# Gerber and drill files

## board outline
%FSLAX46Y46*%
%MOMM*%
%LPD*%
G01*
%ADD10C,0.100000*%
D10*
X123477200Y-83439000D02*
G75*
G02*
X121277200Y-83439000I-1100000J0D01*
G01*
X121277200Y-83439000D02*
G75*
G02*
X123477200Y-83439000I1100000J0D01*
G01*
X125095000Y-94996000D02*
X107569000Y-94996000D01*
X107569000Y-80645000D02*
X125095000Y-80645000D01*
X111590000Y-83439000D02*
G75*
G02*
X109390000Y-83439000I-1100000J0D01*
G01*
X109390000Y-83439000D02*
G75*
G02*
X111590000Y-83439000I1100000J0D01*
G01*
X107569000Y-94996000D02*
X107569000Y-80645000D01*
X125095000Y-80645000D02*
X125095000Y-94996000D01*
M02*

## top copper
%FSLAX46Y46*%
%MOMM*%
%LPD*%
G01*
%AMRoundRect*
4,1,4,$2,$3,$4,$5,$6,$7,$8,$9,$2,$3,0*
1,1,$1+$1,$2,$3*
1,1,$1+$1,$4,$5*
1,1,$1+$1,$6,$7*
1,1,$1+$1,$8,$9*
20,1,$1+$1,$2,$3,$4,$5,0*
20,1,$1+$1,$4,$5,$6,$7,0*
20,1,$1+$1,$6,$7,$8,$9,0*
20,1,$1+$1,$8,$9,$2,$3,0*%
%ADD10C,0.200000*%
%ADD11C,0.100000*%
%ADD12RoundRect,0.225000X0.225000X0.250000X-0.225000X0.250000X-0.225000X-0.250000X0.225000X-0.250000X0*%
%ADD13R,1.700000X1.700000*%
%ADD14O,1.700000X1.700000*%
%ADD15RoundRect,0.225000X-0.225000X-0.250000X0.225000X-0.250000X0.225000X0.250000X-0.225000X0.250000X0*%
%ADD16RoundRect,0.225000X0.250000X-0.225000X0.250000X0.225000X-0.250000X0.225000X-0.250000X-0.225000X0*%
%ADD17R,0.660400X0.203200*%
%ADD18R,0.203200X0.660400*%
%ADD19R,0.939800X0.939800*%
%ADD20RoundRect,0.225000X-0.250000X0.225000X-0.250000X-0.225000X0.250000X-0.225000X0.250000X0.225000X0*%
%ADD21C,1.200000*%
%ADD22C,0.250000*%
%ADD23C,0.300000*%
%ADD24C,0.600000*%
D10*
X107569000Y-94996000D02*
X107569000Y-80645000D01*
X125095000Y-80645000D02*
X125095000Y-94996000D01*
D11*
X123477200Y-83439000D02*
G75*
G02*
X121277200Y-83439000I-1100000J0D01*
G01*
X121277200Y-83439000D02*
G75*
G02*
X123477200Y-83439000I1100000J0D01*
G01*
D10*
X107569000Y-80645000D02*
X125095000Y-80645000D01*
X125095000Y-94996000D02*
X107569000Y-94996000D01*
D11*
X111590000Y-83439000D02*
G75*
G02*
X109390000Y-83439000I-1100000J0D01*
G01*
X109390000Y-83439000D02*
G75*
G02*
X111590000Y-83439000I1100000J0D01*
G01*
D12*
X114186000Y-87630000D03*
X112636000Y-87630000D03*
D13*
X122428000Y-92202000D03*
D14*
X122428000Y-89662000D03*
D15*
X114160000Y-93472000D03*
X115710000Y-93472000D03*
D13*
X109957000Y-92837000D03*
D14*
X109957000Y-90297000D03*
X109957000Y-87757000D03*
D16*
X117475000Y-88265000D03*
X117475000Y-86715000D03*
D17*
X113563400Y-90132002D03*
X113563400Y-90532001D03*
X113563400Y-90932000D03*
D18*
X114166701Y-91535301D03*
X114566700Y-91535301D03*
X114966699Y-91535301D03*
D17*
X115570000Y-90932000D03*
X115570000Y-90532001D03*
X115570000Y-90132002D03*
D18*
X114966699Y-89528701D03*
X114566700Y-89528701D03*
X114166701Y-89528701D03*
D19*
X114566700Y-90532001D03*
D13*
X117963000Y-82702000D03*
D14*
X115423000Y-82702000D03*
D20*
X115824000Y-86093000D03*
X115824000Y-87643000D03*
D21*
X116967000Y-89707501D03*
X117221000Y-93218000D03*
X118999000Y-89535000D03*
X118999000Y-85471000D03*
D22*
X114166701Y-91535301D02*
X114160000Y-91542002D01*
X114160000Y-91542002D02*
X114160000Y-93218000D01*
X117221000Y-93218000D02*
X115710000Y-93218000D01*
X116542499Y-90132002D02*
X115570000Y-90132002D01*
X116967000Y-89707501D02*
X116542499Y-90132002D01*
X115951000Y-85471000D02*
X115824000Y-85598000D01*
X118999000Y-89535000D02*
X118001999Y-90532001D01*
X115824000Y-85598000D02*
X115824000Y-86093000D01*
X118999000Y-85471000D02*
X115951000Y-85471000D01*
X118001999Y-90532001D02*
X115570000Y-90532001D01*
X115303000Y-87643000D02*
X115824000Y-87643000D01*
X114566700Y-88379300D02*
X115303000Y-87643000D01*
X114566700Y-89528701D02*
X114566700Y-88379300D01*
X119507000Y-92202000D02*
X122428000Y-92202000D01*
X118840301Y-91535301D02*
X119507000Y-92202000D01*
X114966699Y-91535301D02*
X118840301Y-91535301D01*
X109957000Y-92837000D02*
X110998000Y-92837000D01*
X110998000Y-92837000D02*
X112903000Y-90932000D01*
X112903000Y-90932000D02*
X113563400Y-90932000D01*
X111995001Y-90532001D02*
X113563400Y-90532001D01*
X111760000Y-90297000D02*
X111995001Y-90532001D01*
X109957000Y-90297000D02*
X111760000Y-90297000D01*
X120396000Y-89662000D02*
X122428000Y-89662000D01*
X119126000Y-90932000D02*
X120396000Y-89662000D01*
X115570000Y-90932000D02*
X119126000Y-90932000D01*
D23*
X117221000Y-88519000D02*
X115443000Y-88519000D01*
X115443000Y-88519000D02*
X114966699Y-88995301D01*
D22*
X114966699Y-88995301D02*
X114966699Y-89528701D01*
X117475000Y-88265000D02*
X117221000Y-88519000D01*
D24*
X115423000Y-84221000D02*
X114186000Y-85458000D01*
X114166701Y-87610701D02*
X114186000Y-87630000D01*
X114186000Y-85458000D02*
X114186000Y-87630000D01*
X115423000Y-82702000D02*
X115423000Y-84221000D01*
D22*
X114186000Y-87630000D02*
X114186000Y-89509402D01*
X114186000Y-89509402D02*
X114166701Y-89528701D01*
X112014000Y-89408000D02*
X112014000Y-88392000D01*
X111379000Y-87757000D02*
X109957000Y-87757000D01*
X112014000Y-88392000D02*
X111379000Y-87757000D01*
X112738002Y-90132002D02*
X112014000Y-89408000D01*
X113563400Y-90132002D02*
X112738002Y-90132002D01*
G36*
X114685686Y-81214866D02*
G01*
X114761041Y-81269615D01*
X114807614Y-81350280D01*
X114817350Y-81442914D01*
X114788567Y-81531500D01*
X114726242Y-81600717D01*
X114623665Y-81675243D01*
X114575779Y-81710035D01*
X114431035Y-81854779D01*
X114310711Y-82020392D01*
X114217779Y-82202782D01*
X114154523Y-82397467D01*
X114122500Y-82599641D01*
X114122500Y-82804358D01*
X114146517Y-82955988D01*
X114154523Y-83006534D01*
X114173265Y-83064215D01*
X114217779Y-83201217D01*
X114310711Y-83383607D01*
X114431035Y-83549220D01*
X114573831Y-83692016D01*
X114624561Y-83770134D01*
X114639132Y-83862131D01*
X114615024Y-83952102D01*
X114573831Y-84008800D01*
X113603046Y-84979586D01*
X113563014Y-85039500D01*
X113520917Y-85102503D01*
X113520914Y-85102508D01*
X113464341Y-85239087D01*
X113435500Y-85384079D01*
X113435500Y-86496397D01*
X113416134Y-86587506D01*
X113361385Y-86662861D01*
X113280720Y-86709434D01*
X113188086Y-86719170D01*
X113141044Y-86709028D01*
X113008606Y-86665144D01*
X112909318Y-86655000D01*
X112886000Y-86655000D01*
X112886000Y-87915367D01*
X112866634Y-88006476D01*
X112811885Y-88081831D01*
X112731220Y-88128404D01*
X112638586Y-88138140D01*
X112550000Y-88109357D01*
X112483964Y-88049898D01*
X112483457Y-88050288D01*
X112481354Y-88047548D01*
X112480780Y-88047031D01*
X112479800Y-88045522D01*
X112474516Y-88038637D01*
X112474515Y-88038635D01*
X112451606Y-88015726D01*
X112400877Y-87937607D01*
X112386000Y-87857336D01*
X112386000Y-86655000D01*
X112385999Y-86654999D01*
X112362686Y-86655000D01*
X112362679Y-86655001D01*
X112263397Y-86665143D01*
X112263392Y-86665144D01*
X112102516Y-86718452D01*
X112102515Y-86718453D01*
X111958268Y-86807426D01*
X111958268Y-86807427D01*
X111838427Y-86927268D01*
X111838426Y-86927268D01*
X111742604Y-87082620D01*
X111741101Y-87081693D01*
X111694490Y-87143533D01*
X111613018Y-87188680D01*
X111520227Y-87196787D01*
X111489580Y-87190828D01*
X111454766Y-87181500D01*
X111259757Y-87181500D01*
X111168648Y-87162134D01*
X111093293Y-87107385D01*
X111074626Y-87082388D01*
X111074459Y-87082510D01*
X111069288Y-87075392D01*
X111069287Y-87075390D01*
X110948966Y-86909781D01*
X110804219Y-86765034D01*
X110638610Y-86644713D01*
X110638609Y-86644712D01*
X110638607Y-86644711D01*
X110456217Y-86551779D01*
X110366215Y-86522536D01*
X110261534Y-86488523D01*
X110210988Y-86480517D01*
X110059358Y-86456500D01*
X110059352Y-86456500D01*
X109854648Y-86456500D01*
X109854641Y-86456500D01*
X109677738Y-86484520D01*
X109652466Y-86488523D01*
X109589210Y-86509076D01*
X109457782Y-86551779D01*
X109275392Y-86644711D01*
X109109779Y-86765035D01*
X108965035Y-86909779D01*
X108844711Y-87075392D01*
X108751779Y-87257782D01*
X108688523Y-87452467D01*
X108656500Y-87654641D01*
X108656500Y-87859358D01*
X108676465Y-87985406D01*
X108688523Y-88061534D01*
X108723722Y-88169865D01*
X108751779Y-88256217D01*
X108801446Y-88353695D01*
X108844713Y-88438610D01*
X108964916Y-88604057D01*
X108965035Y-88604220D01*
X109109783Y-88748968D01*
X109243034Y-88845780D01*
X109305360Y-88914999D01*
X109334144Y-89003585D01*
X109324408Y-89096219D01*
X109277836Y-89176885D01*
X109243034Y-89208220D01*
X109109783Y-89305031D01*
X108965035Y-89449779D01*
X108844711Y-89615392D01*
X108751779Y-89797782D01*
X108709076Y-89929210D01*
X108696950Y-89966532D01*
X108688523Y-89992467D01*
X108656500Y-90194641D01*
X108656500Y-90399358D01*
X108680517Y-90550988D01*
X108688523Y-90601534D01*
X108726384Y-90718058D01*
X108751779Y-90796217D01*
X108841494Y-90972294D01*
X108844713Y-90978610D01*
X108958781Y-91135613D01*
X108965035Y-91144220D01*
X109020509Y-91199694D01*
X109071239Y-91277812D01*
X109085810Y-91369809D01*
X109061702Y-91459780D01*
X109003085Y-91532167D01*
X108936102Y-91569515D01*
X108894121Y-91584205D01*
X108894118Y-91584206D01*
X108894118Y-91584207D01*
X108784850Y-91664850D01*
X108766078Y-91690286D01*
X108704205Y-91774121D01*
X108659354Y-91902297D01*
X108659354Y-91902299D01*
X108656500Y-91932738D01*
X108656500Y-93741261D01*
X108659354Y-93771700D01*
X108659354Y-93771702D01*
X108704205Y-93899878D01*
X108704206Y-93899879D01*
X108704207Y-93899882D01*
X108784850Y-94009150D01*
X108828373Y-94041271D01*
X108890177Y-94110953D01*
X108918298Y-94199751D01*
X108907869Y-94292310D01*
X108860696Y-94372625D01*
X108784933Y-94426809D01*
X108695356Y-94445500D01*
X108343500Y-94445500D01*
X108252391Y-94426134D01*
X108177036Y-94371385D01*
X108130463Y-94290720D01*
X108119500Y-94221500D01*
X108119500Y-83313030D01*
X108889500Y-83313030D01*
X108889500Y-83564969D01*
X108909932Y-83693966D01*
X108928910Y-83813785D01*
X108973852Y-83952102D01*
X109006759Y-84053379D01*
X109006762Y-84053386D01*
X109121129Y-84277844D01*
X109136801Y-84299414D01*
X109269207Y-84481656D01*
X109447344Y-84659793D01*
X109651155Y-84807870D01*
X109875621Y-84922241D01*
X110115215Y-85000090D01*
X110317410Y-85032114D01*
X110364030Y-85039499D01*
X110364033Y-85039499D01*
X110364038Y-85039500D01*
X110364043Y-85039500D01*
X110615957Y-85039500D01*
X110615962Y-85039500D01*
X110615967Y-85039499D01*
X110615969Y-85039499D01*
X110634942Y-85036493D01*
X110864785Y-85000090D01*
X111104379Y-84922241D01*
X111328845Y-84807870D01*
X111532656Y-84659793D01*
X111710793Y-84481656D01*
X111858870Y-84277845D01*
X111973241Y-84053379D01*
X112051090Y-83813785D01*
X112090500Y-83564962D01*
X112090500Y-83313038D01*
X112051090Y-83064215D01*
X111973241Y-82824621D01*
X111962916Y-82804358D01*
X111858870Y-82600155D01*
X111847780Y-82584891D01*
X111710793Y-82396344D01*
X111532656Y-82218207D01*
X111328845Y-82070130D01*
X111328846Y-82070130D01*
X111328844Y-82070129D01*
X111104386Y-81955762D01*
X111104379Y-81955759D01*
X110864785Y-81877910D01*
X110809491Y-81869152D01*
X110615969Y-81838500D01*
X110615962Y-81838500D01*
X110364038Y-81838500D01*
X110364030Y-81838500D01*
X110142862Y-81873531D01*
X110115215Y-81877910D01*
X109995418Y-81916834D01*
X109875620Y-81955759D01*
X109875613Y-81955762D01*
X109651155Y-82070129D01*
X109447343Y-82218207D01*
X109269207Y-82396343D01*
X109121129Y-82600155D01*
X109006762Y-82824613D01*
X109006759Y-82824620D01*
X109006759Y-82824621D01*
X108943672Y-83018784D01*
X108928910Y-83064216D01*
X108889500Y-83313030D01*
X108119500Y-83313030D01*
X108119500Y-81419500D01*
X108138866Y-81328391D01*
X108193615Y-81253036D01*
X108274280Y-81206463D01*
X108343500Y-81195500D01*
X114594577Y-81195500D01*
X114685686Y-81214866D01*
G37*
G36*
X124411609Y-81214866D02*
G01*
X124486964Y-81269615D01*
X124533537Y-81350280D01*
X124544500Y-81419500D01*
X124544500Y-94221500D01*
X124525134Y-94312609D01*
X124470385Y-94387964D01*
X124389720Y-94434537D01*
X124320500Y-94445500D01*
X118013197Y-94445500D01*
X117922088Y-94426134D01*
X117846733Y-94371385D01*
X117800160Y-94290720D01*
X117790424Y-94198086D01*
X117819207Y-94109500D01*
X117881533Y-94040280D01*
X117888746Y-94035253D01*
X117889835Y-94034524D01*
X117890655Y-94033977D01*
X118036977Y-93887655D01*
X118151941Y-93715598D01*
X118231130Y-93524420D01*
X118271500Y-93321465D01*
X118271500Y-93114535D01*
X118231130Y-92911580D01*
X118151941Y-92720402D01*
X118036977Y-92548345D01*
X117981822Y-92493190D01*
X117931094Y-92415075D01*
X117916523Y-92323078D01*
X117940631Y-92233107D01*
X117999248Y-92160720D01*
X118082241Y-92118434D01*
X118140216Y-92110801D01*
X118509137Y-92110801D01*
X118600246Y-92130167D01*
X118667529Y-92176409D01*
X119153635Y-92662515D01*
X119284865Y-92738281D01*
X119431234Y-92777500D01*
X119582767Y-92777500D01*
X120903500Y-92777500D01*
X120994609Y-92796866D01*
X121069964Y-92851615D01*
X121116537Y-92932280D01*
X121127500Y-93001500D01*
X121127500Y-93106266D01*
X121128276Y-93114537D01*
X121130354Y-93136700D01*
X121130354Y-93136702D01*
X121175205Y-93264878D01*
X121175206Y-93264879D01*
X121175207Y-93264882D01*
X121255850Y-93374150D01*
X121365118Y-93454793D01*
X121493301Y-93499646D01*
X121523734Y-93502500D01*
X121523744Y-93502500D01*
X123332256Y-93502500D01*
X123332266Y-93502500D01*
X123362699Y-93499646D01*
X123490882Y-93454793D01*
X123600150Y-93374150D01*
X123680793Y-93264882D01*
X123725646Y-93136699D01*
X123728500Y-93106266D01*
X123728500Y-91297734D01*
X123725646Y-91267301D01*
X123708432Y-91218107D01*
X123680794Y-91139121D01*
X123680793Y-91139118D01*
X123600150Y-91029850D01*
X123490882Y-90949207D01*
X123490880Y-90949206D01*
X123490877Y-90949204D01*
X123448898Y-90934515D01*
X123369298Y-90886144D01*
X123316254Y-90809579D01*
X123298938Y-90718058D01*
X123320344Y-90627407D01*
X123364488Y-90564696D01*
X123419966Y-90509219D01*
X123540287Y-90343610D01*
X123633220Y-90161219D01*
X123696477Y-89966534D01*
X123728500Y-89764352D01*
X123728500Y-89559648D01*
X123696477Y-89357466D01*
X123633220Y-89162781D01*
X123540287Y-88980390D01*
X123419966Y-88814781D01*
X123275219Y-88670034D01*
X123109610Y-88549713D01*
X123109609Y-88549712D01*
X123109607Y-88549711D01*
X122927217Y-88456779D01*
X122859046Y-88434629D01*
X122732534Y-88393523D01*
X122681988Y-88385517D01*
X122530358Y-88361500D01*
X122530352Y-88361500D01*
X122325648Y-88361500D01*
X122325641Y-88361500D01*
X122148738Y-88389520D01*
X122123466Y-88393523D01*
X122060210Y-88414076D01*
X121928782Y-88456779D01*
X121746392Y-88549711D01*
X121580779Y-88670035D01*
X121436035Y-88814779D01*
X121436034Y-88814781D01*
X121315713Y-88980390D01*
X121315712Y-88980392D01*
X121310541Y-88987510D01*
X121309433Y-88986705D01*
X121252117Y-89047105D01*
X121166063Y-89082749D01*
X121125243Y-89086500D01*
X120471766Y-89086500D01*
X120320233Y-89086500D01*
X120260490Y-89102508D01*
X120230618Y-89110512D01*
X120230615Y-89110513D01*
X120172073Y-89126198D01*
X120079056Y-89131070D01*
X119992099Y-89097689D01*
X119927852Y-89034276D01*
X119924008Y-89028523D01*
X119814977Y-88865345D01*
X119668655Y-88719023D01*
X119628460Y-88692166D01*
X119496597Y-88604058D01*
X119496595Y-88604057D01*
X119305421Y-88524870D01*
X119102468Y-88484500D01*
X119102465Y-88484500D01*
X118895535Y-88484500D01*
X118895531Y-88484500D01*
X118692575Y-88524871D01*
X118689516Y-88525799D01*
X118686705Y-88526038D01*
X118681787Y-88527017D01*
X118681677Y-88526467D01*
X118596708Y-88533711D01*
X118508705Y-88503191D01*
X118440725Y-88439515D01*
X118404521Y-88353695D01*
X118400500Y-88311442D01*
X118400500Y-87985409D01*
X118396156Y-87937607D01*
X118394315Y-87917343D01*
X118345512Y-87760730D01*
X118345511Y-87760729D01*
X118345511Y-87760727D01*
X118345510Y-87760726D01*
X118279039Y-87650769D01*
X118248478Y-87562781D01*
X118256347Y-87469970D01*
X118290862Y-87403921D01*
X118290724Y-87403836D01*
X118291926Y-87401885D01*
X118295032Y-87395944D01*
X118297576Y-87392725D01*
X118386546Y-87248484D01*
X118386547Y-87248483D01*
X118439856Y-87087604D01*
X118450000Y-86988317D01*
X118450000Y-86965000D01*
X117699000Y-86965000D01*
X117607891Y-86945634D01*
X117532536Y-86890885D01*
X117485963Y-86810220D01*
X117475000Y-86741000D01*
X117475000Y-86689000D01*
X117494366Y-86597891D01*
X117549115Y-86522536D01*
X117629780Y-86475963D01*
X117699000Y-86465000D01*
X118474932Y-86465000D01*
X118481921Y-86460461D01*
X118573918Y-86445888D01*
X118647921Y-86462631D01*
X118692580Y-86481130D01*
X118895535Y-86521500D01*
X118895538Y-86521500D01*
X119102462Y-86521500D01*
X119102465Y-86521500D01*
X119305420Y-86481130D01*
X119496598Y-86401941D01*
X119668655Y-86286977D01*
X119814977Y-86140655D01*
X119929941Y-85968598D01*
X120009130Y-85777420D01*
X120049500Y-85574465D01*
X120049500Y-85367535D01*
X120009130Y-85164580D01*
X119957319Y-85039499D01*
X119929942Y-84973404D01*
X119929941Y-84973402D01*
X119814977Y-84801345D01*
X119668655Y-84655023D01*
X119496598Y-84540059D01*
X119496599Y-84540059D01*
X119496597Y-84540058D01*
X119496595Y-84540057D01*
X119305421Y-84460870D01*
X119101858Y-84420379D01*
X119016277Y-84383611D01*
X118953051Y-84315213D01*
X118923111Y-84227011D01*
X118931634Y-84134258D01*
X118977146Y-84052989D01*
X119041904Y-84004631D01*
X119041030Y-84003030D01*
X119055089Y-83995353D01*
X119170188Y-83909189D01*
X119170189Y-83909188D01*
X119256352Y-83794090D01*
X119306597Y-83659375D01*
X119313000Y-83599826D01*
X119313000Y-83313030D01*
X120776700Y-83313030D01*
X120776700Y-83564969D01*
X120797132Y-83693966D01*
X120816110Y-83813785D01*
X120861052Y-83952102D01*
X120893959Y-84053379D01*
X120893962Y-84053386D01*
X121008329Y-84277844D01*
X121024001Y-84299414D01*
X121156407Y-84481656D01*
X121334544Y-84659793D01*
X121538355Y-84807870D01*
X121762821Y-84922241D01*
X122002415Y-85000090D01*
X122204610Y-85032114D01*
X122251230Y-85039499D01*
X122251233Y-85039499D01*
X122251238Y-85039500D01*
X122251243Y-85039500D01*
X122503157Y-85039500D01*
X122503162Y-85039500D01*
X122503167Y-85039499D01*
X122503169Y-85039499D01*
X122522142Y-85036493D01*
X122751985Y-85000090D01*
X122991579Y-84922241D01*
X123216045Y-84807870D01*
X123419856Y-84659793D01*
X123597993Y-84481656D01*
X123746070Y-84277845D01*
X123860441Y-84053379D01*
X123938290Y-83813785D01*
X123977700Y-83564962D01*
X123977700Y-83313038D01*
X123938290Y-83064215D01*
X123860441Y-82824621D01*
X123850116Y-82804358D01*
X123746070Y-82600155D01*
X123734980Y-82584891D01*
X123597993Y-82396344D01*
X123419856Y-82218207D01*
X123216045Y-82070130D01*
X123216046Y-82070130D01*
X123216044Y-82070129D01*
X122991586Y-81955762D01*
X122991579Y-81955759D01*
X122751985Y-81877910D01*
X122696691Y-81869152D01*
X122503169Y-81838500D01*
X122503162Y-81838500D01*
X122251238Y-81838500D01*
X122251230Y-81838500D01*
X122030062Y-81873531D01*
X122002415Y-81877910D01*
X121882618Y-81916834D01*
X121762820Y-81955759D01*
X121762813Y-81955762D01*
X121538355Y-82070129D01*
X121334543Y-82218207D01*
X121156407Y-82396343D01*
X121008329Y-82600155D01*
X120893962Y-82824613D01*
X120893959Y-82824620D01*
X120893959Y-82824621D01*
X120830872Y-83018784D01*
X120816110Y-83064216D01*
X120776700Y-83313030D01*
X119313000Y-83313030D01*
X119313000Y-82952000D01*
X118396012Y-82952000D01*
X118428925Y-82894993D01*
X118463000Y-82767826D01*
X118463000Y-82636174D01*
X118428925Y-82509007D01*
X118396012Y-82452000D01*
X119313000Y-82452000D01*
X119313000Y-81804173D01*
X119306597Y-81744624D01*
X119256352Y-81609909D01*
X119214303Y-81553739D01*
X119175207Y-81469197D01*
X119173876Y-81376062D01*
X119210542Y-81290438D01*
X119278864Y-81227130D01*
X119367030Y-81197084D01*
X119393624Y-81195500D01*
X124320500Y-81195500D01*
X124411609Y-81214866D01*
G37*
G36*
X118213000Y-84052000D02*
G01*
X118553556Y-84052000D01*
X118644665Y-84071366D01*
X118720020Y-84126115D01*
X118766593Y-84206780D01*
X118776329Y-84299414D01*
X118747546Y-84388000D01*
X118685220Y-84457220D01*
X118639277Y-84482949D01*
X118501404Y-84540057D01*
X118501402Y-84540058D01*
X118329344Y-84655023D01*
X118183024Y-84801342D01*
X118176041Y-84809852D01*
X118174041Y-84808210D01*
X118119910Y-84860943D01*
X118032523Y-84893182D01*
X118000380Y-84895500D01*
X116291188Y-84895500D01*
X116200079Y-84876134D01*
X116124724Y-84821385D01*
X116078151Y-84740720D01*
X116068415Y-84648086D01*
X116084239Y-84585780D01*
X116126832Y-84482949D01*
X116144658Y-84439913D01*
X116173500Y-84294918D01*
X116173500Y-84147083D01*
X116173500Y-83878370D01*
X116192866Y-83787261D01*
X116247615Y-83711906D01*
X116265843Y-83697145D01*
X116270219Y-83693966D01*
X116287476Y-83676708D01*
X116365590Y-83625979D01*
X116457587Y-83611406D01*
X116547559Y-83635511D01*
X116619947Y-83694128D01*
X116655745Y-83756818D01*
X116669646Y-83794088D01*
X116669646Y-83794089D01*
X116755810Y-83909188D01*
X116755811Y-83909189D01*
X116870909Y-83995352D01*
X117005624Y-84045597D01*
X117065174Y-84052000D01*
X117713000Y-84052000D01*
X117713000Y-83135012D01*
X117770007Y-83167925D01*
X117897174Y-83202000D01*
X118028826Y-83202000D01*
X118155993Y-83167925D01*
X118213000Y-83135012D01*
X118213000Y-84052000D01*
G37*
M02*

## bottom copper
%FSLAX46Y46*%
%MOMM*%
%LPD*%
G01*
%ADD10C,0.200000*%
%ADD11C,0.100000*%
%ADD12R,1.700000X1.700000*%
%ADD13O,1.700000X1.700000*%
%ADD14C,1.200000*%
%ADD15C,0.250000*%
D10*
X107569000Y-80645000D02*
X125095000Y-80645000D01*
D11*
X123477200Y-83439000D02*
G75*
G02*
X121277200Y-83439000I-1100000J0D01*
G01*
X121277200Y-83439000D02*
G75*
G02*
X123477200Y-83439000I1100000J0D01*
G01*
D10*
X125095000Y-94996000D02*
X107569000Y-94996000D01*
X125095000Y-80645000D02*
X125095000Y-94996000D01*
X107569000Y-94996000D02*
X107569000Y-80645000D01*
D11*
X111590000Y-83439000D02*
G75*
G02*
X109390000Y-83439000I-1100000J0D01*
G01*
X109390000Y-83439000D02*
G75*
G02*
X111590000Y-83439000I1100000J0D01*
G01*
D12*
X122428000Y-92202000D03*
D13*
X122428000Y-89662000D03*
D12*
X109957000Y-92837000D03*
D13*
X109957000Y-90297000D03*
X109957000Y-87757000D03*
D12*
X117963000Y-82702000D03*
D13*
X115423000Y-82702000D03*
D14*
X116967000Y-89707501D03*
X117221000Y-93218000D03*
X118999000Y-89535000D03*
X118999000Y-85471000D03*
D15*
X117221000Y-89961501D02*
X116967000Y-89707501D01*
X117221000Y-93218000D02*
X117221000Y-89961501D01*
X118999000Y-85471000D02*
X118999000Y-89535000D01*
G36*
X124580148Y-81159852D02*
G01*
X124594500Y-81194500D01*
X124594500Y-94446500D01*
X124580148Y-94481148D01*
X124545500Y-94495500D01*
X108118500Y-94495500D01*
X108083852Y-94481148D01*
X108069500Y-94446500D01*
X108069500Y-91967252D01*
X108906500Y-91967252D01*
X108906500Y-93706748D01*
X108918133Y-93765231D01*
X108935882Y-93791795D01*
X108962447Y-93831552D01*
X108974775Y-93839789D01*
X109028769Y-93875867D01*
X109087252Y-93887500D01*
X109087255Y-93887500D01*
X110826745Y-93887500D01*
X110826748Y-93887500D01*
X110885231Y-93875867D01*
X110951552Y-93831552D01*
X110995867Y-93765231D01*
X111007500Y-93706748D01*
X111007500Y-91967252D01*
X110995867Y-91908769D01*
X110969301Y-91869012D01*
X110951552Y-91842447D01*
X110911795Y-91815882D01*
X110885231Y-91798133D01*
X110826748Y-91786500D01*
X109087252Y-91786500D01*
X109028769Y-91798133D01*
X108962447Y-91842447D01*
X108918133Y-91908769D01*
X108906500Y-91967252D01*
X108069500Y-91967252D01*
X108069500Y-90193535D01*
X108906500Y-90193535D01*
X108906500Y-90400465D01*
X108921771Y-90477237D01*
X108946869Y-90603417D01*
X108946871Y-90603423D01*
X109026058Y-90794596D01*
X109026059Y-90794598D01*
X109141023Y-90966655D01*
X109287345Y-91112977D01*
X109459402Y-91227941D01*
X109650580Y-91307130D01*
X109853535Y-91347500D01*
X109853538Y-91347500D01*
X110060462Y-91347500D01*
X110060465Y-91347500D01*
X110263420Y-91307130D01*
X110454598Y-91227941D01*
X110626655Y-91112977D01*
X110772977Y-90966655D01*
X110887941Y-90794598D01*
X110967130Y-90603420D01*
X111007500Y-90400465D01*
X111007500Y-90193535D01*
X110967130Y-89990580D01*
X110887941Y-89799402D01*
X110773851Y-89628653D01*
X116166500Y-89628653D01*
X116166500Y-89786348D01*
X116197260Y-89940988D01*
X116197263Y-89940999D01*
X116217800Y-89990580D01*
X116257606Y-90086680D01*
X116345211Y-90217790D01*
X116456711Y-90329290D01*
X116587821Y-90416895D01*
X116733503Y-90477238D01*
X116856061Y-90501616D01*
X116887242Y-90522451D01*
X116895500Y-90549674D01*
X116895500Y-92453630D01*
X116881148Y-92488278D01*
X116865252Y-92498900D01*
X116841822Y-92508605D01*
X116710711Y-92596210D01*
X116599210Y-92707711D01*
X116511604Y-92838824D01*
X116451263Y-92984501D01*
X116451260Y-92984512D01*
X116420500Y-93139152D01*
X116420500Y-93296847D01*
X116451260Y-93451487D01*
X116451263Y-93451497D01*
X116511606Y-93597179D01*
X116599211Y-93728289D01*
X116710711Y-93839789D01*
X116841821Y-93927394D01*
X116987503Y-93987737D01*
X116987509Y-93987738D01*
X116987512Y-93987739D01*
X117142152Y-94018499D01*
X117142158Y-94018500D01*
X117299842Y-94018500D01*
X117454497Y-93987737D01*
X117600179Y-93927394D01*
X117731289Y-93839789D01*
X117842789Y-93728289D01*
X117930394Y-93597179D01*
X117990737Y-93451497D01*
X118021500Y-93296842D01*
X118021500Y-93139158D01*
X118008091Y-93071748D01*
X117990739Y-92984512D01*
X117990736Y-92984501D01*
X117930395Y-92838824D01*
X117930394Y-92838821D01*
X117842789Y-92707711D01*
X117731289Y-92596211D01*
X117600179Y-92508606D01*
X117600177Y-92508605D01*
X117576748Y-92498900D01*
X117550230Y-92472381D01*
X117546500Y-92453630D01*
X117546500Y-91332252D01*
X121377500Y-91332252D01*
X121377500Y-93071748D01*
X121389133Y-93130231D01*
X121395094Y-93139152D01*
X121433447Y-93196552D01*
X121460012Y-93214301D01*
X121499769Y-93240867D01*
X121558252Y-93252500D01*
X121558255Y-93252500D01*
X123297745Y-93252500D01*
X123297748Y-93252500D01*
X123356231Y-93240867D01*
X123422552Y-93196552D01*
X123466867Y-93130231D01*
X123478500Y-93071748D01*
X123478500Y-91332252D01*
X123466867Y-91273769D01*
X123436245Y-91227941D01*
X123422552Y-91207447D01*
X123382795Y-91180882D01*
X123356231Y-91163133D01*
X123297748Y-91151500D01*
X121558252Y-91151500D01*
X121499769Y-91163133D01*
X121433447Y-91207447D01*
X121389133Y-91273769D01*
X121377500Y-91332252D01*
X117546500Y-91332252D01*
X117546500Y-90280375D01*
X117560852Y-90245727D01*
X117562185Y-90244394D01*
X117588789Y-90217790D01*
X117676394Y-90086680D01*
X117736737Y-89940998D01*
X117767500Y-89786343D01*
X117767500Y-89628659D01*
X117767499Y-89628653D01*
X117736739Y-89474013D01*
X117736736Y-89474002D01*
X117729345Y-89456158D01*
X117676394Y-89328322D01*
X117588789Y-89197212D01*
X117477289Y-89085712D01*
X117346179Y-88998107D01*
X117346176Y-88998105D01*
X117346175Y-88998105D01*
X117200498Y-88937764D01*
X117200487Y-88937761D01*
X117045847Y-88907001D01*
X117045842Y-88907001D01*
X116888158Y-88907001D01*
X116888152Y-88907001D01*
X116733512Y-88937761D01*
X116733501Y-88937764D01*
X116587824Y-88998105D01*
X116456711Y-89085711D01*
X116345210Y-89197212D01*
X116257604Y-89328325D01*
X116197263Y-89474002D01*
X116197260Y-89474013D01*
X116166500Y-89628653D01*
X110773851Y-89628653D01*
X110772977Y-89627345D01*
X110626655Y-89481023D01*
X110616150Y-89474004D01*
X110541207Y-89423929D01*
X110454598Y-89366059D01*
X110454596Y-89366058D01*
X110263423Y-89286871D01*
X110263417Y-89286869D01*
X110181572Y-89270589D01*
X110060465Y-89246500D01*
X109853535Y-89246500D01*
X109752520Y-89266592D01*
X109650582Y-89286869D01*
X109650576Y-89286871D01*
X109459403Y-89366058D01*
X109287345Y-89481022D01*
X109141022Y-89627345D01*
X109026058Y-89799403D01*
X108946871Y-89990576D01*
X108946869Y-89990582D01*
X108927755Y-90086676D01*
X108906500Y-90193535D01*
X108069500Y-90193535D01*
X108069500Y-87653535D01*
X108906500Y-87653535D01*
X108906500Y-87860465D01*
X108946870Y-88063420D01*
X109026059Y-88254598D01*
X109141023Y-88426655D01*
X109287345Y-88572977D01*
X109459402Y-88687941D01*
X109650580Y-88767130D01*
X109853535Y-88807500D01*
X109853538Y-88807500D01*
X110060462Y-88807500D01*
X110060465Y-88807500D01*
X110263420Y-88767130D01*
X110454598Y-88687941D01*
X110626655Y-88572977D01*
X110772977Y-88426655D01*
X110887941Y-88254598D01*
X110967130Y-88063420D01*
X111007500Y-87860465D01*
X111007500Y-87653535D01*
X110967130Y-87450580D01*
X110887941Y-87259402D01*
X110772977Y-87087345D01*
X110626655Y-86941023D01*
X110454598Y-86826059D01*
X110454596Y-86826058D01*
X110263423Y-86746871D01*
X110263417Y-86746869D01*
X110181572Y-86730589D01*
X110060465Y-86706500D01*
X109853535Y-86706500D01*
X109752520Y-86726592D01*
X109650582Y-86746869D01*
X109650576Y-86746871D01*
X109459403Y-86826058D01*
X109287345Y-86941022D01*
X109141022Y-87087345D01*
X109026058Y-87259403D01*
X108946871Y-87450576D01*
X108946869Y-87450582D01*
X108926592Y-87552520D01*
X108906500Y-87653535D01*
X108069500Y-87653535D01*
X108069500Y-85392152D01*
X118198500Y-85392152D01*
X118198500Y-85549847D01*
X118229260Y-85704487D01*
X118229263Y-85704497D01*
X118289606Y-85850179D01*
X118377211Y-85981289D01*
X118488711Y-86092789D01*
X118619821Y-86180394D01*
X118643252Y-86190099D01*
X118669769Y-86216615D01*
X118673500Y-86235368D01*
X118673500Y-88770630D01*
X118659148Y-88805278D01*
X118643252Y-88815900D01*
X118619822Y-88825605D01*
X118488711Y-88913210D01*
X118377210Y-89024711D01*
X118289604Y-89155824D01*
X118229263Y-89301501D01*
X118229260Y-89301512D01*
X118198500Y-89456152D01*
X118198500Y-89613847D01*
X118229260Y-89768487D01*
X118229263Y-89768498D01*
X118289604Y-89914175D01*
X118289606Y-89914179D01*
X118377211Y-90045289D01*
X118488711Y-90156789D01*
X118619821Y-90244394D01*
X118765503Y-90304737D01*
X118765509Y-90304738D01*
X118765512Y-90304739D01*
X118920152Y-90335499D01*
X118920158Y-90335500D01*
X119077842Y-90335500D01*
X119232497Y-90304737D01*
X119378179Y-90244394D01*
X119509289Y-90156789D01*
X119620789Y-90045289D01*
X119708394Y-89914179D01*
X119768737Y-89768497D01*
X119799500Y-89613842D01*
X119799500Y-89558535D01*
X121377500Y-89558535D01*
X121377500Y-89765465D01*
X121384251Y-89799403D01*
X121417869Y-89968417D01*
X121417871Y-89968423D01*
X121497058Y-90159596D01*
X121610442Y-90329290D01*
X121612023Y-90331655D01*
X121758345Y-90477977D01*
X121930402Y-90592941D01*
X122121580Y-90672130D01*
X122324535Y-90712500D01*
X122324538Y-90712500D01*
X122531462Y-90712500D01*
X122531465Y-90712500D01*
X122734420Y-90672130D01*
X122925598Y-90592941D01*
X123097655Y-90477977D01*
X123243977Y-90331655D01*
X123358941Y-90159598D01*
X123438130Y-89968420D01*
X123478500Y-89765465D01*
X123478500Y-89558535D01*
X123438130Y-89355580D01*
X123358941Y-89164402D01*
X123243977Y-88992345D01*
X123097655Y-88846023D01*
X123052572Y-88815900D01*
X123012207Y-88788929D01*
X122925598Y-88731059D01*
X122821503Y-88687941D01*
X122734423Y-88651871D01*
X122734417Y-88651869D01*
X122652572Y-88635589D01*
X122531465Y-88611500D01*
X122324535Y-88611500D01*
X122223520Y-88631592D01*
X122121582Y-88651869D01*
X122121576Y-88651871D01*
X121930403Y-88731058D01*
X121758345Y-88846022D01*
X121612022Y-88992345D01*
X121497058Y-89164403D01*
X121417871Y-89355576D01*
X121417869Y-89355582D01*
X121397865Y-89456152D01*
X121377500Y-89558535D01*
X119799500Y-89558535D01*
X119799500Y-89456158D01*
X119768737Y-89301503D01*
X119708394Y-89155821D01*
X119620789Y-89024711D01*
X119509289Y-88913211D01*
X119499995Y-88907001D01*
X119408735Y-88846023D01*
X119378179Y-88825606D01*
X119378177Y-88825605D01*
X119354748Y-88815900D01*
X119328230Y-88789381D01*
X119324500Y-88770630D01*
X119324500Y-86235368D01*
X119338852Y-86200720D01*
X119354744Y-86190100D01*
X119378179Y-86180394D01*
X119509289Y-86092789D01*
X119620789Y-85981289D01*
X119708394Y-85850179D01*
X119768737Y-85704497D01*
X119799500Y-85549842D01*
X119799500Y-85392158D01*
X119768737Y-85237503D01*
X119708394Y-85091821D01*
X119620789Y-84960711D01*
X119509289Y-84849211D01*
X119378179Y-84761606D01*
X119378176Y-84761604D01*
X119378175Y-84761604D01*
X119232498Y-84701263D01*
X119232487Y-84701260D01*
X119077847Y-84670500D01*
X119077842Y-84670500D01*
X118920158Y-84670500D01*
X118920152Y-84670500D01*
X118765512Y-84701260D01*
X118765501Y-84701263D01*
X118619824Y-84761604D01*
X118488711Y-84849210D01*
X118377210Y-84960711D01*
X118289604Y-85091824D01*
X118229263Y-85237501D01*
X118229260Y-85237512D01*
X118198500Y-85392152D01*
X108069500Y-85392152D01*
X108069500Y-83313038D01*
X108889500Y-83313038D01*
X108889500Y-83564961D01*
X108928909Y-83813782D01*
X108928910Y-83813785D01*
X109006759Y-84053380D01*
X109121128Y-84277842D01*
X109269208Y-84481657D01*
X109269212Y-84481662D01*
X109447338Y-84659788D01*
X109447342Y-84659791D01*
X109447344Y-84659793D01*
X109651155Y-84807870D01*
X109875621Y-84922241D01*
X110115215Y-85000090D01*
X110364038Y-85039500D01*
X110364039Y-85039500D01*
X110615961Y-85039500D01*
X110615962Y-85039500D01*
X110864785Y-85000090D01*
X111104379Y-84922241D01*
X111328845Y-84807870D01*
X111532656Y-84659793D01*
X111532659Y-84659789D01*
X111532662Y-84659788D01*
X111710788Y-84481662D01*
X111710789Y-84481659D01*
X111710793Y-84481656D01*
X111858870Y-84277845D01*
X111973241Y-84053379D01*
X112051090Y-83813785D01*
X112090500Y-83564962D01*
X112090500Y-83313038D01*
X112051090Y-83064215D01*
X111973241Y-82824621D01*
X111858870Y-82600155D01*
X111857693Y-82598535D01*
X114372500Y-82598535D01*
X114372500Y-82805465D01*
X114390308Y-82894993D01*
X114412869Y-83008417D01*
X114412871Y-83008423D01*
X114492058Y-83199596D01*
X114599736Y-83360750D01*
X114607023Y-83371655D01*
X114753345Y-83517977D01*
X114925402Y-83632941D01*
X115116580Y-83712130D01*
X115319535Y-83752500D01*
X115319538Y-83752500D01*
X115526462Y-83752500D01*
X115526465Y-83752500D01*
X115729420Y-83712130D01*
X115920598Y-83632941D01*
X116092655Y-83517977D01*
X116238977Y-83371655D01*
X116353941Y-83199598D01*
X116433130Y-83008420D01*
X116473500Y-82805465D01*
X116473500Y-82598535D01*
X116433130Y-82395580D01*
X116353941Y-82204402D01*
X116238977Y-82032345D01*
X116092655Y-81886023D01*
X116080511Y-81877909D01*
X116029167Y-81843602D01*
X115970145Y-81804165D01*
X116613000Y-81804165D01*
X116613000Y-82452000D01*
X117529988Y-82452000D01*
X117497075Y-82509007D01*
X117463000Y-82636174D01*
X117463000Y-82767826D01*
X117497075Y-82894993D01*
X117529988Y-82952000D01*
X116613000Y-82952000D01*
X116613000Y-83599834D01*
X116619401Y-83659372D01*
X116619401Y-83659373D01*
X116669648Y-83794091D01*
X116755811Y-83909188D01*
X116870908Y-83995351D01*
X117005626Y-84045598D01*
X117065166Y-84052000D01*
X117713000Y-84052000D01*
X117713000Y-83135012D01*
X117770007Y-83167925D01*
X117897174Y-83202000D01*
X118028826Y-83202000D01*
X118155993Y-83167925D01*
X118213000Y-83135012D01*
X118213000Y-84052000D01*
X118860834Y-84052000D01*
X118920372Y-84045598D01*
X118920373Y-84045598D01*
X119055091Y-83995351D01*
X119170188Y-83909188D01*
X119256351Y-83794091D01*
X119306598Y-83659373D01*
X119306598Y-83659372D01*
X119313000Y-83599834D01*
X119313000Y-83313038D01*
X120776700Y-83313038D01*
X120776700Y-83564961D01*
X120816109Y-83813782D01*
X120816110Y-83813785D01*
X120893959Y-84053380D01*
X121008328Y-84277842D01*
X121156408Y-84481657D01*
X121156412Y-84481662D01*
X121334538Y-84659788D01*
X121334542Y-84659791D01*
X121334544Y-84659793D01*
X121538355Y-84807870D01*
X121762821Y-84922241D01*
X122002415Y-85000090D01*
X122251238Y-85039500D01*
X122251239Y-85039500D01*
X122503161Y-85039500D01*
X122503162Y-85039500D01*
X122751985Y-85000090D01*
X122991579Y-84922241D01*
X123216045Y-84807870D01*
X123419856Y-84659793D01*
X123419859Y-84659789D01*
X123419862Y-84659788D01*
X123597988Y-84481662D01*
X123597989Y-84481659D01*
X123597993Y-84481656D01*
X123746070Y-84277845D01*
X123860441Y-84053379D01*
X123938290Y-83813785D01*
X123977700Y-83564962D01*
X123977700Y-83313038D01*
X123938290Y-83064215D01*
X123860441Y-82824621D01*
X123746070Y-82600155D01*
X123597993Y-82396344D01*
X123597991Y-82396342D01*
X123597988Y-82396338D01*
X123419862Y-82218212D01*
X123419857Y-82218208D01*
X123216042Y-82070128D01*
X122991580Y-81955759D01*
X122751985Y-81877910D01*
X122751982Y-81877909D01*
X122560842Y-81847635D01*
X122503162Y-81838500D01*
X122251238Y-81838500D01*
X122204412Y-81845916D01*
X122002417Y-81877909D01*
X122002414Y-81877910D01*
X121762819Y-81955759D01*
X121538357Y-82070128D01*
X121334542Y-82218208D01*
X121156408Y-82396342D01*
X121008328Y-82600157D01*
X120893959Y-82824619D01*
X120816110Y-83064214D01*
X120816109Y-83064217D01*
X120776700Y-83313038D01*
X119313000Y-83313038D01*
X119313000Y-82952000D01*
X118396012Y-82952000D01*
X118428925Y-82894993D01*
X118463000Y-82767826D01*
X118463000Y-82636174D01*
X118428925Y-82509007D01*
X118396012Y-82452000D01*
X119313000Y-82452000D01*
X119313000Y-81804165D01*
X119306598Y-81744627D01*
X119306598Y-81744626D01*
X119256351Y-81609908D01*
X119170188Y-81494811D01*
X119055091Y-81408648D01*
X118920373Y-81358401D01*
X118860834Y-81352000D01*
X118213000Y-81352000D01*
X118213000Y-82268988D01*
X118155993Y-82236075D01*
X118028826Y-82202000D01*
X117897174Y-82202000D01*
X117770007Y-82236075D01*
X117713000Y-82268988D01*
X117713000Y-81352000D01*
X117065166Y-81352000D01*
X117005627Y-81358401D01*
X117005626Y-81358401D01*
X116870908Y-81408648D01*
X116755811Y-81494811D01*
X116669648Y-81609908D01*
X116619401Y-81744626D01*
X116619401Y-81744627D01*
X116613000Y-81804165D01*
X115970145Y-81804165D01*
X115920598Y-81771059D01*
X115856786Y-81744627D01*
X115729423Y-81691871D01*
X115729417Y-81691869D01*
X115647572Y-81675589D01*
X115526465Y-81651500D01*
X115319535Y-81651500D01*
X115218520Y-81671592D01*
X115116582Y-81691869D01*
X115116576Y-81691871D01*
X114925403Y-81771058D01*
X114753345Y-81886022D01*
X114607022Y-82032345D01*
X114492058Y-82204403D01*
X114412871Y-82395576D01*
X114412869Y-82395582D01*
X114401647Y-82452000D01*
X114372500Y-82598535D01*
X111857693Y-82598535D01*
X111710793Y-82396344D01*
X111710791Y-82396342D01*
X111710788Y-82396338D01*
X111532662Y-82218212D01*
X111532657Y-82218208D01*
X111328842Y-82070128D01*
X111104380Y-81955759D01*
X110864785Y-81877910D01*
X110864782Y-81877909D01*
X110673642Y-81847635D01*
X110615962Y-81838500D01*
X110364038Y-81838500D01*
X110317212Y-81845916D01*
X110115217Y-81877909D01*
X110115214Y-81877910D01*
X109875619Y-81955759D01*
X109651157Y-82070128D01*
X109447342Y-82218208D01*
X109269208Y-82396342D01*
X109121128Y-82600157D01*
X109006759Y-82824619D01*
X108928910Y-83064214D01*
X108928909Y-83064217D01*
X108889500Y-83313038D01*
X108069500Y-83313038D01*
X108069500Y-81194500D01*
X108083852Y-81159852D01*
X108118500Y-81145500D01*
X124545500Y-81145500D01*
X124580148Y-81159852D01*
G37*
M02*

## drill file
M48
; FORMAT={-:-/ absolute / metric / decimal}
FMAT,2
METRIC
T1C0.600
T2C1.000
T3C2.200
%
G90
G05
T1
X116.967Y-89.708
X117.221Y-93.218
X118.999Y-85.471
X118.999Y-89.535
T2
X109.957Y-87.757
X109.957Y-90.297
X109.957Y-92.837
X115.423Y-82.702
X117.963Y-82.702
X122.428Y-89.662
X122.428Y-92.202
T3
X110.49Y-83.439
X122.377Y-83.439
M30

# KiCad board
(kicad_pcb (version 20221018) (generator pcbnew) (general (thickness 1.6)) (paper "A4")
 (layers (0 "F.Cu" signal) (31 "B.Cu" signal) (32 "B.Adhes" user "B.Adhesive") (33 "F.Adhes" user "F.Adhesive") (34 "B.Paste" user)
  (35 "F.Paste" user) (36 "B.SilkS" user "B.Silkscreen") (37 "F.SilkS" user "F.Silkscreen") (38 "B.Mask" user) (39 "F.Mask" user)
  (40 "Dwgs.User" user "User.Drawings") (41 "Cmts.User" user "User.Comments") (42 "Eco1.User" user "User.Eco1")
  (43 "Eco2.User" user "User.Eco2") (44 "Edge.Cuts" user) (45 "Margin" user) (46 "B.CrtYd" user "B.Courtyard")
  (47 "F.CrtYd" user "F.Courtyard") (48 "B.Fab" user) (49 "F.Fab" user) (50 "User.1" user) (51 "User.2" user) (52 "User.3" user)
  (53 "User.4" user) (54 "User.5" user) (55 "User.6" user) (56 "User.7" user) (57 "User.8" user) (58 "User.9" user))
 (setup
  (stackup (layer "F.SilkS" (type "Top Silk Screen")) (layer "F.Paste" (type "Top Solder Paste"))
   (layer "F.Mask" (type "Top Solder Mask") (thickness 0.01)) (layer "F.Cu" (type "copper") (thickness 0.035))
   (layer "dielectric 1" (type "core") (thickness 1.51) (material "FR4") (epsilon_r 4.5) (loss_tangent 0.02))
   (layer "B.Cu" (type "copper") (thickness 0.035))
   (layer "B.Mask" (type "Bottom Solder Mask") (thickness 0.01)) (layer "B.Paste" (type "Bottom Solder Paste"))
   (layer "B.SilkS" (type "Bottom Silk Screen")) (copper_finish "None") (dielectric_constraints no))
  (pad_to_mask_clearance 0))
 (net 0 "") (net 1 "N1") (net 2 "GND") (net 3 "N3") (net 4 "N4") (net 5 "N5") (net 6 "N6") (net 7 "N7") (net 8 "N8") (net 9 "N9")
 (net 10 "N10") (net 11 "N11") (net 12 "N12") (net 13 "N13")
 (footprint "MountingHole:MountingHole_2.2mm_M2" (layer "F.Cu") (at 122.3772 83.439)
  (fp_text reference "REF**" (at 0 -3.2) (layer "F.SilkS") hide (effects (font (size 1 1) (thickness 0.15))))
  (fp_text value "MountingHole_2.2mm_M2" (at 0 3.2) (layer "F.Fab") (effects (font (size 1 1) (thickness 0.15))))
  (pad "" np_thru_hole circle (at 0 0) (size 2.2 2.2) (drill 2.2) (layers "F&B.Cu" "*.Mask")))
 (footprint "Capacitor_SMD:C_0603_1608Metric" (layer "F.Cu") (at 113.411 87.63 180)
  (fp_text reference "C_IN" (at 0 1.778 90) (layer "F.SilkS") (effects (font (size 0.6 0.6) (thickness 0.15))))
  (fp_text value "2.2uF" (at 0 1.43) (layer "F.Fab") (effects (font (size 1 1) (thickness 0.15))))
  (pad "1" smd roundrect (at -0.775 0 180) (size 0.9 0.95) (layers "F.Cu" "F.Paste" "F.Mask") (roundrect_rratio 0.25) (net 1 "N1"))
  (pad "2" smd roundrect (at 0.775 0 180) (size 0.9 0.95) (layers "F.Cu" "F.Paste" "F.Mask") (roundrect_rratio 0.25) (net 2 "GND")))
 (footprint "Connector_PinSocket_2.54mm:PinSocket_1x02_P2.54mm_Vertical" (layer "F.Cu") (at 122.428 92.202 180)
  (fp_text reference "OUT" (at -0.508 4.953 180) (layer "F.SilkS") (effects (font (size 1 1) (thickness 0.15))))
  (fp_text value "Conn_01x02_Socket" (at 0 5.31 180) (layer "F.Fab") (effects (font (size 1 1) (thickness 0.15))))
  (pad "1" thru_hole rect (at 0 0 180) (size 1.7 1.7) (drill 1) (layers "*.Cu" "*.Mask") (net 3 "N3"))
  (pad "2" thru_hole oval (at 0 2.54 180) (size 1.7 1.7) (drill 1) (layers "*.Cu" "*.Mask") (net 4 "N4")))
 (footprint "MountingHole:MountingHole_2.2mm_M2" (layer "F.Cu") (at 110.49 83.439)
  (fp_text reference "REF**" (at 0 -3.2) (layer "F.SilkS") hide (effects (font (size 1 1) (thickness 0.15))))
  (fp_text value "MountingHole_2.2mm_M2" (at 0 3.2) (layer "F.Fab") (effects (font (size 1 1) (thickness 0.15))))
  (pad "" np_thru_hole circle (at 0 0) (size 2.2 2.2) (drill 2.2) (layers "*.Cu" "*.Mask")))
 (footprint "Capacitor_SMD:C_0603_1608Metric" (layer "F.Cu") (at 114.935 93.472)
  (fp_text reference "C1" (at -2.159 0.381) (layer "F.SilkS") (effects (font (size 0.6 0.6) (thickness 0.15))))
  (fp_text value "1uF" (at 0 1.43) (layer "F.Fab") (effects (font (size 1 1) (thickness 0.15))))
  (pad "1" smd roundrect (at -0.775 0) (size 0.9 0.95) (layers "F.Cu" "F.Paste" "F.Mask") (roundrect_rratio 0.25) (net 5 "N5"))
  (pad "2" smd roundrect (at 0.775 0) (size 0.9 0.95) (layers "F.Cu" "F.Paste" "F.Mask") (roundrect_rratio 0.25) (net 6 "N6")))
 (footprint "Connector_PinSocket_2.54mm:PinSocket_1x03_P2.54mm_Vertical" (layer "F.Cu") (at 109.957 92.837 180)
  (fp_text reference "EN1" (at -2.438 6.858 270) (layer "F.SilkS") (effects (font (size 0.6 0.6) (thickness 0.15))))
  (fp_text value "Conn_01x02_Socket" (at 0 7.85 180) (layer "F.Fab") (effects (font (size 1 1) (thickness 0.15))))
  (pad "1" thru_hole rect (at 0 0 180) (size 1.7 1.7) (drill 1) (layers "*.Cu" "*.Mask") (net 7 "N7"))
  (pad "2" thru_hole oval (at 0 2.54 180) (size 1.7 1.7) (drill 1) (layers "*.Cu" "*.Mask") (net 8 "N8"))
  (pad "3" thru_hole oval (at 0 5.08 180) (size 1.7 1.7) (drill 1) (layers "*.Cu" "*.Mask") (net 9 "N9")))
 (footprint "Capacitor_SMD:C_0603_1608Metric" (layer "F.Cu") (at 117.475 87.49 90)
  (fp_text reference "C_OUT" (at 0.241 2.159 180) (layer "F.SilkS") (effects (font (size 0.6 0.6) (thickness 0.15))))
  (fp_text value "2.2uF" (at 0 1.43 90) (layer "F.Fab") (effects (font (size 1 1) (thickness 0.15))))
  (pad "1" smd roundrect (at -0.775 0 90) (size 0.9 0.95) (layers "F.Cu" "F.Paste" "F.Mask") (roundrect_rratio 0.25) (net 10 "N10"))
  (pad "2" smd roundrect (at 0.775 0 90) (size 0.9 0.95) (layers "F.Cu" "F.Paste" "F.Mask") (roundrect_rratio 0.25) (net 2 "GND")))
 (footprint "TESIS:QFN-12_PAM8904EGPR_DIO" (layer "F.Cu") (at 114.5667 90.532001)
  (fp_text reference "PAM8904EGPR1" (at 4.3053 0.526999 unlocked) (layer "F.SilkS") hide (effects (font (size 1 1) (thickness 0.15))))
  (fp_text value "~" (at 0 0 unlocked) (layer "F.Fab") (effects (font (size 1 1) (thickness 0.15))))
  (pad "1" smd rect (at -1.0033 -0.399999 90) (size 0.2032 0.6604) (layers "F.Cu" "F.Paste" "F.Mask") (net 9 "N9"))
  (pad "2" smd rect (at -1.0033 0 90) (size 0.2032 0.6604) (layers "F.Cu" "F.Paste" "F.Mask") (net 8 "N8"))
  (pad "3" smd rect (at -1.0033 0.399999 90) (size 0.2032 0.6604) (layers "F.Cu" "F.Paste" "F.Mask") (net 7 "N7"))
  (pad "4" smd rect (at -0.399999 1.0033) (size 0.2032 0.6604) (layers "F.Cu" "F.Paste" "F.Mask") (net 5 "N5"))
  (pad "5" smd rect (at 0 1.0033) (size 0.2032 0.6604) (layers "F.Cu" "F.Paste" "F.Mask") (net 2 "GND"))
  (pad "6" smd rect (at 0.399999 1.0033) (size 0.2032 0.6604) (layers "F.Cu" "F.Paste" "F.Mask") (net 3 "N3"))
  (pad "7" smd rect (at 1.0033 0.399999 90) (size 0.2032 0.6604) (layers "F.Cu" "F.Paste" "F.Mask") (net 4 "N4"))
  (pad "8" smd rect (at 1.0033 0 90) (size 0.2032 0.6604) (layers "F.Cu" "F.Paste" "F.Mask") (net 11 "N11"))
  (pad "9" smd rect (at 1.0033 -0.399999 90) (size 0.2032 0.6604) (layers "F.Cu" "F.Paste" "F.Mask") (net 6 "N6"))
  (pad "10" smd rect (at 0.399999 -1.0033) (size 0.2032 0.6604) (layers "F.Cu" "F.Paste" "F.Mask") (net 10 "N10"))
  (pad "11" smd rect (at 0 -1.0033) (size 0.2032 0.6604) (layers "F.Cu" "F.Paste" "F.Mask") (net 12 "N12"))
  (pad "12" smd rect (at -0.399999 -1.0033) (size 0.2032 0.6604) (layers "F.Cu" "F.Paste" "F.Mask") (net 1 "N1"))
  (pad "13" smd rect (at 0 0) (size 0.9398 0.9398) (layers "F.Cu" "F.Paste" "F.Mask") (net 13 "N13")))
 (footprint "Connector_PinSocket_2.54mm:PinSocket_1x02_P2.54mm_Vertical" (layer "F.Cu") (at 117.963 82.702 -90)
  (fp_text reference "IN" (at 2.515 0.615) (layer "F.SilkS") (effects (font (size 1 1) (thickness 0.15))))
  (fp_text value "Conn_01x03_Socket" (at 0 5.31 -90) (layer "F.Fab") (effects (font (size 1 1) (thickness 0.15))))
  (pad "1" thru_hole rect (at 0 0 270) (size 1.7 1.7) (drill 1) (layers "*.Cu" "*.Mask") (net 2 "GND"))
  (pad "2" thru_hole oval (at 0 2.54 270) (size 1.7 1.7) (drill 1) (layers "*.Cu" "*.Mask") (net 1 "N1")))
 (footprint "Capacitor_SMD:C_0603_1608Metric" (layer "F.Cu") (at 115.824 86.868 -90)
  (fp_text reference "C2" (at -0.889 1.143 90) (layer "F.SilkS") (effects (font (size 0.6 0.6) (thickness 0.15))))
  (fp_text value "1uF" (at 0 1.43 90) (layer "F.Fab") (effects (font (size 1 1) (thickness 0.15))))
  (pad "1" smd roundrect (at -0.775 0 270) (size 0.9 0.95) (layers "F.Cu" "F.Paste" "F.Mask") (roundrect_rratio 0.25) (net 11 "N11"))
  (pad "2" smd roundrect (at 0.775 0 270) (size 0.9 0.95) (layers "F.Cu" "F.Paste" "F.Mask") (roundrect_rratio 0.25) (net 12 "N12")))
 (gr_line (start 107.569 94.996) (end 107.569 80.645) (stroke (width 0.2) (type default)) (layer "F.Cu"))
 (gr_line (start 125.095 80.645) (end 125.095 94.996) (stroke (width 0.2) (type default)) (layer "F.Cu"))
 (gr_circle (center 122.3772 83.439) (end 123.4772 83.439) (stroke (width 0.1) (type default)) (fill none) (layer "F.Cu"))
 (gr_line (start 107.569 80.645) (end 125.095 80.645) (stroke (width 0.2) (type default)) (layer "F.Cu"))
 (gr_line (start 125.095 94.996) (end 107.569 94.996) (stroke (width 0.2) (type default)) (layer "F.Cu"))
 (gr_circle (center 110.49 83.439) (end 111.59 83.439) (stroke (width 0.1) (type default)) (fill none) (layer "F.Cu"))
 (gr_line (start 107.569 80.645) (end 125.095 80.645) (stroke (width 0.2) (type default)) (layer "B.Cu"))
 (gr_circle (center 122.3772 83.439) (end 123.4772 83.439) (stroke (width 0.1) (type default)) (fill none) (layer "B.Cu"))
 (gr_line (start 125.095 94.996) (end 107.569 94.996) (stroke (width 0.2) (type default)) (layer "B.Cu"))
 (gr_line (start 125.095 80.645) (end 125.095 94.996) (stroke (width 0.2) (type default)) (layer "B.Cu"))
 (gr_line (start 107.569 94.996) (end 107.569 80.645) (stroke (width 0.2) (type default)) (layer "B.Cu"))
 (gr_circle (center 110.49 83.439) (end 111.59 83.439) (stroke (width 0.1) (type default)) (fill none) (layer "B.Cu"))
 (gr_circle (center 122.3772 83.439) (end 123.4772 83.439) (stroke (width 0.1) (type default)) (fill none) (layer "Edge.Cuts"))
 (gr_line (start 125.095 94.996) (end 107.569 94.996) (stroke (width 0.1) (type default)) (layer "Edge.Cuts"))
 (gr_line (start 107.569 80.645) (end 125.095 80.645) (stroke (width 0.1) (type default)) (layer "Edge.Cuts"))
 (gr_circle (center 110.49 83.439) (end 111.59 83.439) (stroke (width 0.1) (type default)) (fill none) (layer "Edge.Cuts"))
 (gr_line (start 107.569 94.996) (end 107.569 80.645) (stroke (width 0.1) (type default)) (layer "Edge.Cuts"))
 (gr_line (start 125.095 80.645) (end 125.095 94.996) (stroke (width 0.1) (type default)) (layer "Edge.Cuts"))
 (segment (start 114.166701 91.535301) (end 114.16 91.542002) (width 0.25) (layer "F.Cu") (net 5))
 (segment (start 114.16 91.542002) (end 114.16 93.218) (width 0.25) (layer "F.Cu") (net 5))
 (segment (start 117.221 93.218) (end 115.71 93.218) (width 0.25) (layer "F.Cu") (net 6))
 (segment (start 116.542499 90.132002) (end 115.57 90.132002) (width 0.25) (layer "F.Cu") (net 6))
 (segment (start 116.967 89.707501) (end 116.542499 90.132002) (width 0.25) (layer "F.Cu") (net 6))
 (via (at 116.967 89.707501) (size 1.2) (drill 0.6) (layers "F.Cu" "B.Cu") (free) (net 6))
 (via (at 117.221 93.218) (size 1.2) (drill 0.6) (layers "F.Cu" "B.Cu") (free) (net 6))
 (segment (start 117.221 89.961501) (end 116.967 89.707501) (width 0.25) (layer "B.Cu") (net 6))
 (segment (start 117.221 93.218) (end 117.221 89.961501) (width 0.25) (layer "B.Cu") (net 6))
 (segment (start 115.951 85.471) (end 115.824 85.598) (width 0.25) (layer "F.Cu") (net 11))
 (segment (start 118.999 89.535) (end 118.001999 90.532001) (width 0.25) (layer "F.Cu") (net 11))
 (segment (start 115.824 85.598) (end 115.824 86.093) (width 0.25) (layer "F.Cu") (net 11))
 (segment (start 118.999 85.471) (end 115.951 85.471) (width 0.25) (layer "F.Cu") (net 11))
 (segment (start 118.001999 90.532001) (end 115.57 90.532001) (width 0.25) (layer "F.Cu") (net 11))
 (via (at 118.999 89.535) (size 1.2) (drill 0.6) (layers "F.Cu" "B.Cu") (free) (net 11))
 (via (at 118.999 85.471) (size 1.2) (drill 0.6) (layers "F.Cu" "B.Cu") (free) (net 11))
 (segment (start 118.999 85.471) (end 118.999 89.535) (width 0.25) (layer "B.Cu") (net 11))
 (segment (start 115.303 87.643) (end 115.824 87.643) (width 0.25) (layer "F.Cu") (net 12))
 (segment (start 114.5667 88.3793) (end 115.303 87.643) (width 0.25) (layer "F.Cu") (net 12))
 (segment (start 114.5667 89.528701) (end 114.5667 88.3793) (width 0.25) (layer "F.Cu") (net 12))
 (segment (start 119.507 92.202) (end 122.428 92.202) (width 0.25) (layer "F.Cu") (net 3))
 (segment (start 118.840301 91.535301) (end 119.507 92.202) (width 0.25) (layer "F.Cu") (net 3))
 (segment (start 114.966699 91.535301) (end 118.840301 91.535301) (width 0.25) (layer "F.Cu") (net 3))
 (segment (start 109.957 92.837) (end 110.998 92.837) (width 0.25) (layer "F.Cu") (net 7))
 (segment (start 110.998 92.837) (end 112.903 90.932) (width 0.25) (layer "F.Cu") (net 7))
 (segment (start 112.903 90.932) (end 113.5634 90.932) (width 0.25) (layer "F.Cu") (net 7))
 (segment (start 111.995001 90.532001) (end 113.5634 90.532001) (width 0.25) (layer "F.Cu") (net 8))
 (segment (start 111.76 90.297) (end 111.995001 90.532001) (width 0.25) (layer "F.Cu") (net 8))
 (segment (start 109.957 90.297) (end 111.76 90.297) (width 0.25) (layer "F.Cu") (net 8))
 (segment (start 120.396 89.662) (end 122.428 89.662) (width 0.25) (layer "F.Cu") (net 4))
 (segment (start 119.126 90.932) (end 120.396 89.662) (width 0.25) (layer "F.Cu") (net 4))
 (segment (start 115.57 90.932) (end 119.126 90.932) (width 0.25) (layer "F.Cu") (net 4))
 (segment (start 117.221 88.519) (end 115.443 88.519) (width 0.3) (layer "F.Cu") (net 10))
 (segment (start 115.443 88.519) (end 114.966699 88.995301) (width 0.3) (layer "F.Cu") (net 10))
 (segment (start 114.966699 88.995301) (end 114.966699 89.528701) (width 0.25) (layer "F.Cu") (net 10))
 (segment (start 117.475 88.265) (end 117.221 88.519) (width 0.25) (layer "F.Cu") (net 10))
 (segment (start 115.423 84.221) (end 114.186 85.458) (width 0.6) (layer "F.Cu") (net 1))
 (segment (start 114.166701 87.610701) (end 114.186 87.63) (width 0.6) (layer "F.Cu") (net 1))
 (segment (start 114.186 85.458) (end 114.186 87.63) (width 0.6) (layer "F.Cu") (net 1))
 (segment (start 115.423 82.702) (end 115.423 84.221) (width 0.6) (layer "F.Cu") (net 1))
 (segment (start 114.186 87.63) (end 114.186 89.509402) (width 0.25) (layer "F.Cu") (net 1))
 (segment (start 114.186 89.509402) (end 114.166701 89.528701) (width 0.25) (layer "F.Cu") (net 1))
 (segment (start 112.014 89.408) (end 112.014 88.392) (width 0.25) (layer "F.Cu") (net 9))
 (segment (start 111.379 87.757) (end 109.957 87.757) (width 0.25) (layer "F.Cu") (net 9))
 (segment (start 112.014 88.392) (end 111.379 87.757) (width 0.25) (layer "F.Cu") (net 9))
 (segment (start 112.738002 90.132002) (end 112.014 89.408) (width 0.25) (layer "F.Cu") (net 9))
 (segment (start 113.5634 90.132002) (end 112.738002 90.132002) (width 0.25) (layer "F.Cu") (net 9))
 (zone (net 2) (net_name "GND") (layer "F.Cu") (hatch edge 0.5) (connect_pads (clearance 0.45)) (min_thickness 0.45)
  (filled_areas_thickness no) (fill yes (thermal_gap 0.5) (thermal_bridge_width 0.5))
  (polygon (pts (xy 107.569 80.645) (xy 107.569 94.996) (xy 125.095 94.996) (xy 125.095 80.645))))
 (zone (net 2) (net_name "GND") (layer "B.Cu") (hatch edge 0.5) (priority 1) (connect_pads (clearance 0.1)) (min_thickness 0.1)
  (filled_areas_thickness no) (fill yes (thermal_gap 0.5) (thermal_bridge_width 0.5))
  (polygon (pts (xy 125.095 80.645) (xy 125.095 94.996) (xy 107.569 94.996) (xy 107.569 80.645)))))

